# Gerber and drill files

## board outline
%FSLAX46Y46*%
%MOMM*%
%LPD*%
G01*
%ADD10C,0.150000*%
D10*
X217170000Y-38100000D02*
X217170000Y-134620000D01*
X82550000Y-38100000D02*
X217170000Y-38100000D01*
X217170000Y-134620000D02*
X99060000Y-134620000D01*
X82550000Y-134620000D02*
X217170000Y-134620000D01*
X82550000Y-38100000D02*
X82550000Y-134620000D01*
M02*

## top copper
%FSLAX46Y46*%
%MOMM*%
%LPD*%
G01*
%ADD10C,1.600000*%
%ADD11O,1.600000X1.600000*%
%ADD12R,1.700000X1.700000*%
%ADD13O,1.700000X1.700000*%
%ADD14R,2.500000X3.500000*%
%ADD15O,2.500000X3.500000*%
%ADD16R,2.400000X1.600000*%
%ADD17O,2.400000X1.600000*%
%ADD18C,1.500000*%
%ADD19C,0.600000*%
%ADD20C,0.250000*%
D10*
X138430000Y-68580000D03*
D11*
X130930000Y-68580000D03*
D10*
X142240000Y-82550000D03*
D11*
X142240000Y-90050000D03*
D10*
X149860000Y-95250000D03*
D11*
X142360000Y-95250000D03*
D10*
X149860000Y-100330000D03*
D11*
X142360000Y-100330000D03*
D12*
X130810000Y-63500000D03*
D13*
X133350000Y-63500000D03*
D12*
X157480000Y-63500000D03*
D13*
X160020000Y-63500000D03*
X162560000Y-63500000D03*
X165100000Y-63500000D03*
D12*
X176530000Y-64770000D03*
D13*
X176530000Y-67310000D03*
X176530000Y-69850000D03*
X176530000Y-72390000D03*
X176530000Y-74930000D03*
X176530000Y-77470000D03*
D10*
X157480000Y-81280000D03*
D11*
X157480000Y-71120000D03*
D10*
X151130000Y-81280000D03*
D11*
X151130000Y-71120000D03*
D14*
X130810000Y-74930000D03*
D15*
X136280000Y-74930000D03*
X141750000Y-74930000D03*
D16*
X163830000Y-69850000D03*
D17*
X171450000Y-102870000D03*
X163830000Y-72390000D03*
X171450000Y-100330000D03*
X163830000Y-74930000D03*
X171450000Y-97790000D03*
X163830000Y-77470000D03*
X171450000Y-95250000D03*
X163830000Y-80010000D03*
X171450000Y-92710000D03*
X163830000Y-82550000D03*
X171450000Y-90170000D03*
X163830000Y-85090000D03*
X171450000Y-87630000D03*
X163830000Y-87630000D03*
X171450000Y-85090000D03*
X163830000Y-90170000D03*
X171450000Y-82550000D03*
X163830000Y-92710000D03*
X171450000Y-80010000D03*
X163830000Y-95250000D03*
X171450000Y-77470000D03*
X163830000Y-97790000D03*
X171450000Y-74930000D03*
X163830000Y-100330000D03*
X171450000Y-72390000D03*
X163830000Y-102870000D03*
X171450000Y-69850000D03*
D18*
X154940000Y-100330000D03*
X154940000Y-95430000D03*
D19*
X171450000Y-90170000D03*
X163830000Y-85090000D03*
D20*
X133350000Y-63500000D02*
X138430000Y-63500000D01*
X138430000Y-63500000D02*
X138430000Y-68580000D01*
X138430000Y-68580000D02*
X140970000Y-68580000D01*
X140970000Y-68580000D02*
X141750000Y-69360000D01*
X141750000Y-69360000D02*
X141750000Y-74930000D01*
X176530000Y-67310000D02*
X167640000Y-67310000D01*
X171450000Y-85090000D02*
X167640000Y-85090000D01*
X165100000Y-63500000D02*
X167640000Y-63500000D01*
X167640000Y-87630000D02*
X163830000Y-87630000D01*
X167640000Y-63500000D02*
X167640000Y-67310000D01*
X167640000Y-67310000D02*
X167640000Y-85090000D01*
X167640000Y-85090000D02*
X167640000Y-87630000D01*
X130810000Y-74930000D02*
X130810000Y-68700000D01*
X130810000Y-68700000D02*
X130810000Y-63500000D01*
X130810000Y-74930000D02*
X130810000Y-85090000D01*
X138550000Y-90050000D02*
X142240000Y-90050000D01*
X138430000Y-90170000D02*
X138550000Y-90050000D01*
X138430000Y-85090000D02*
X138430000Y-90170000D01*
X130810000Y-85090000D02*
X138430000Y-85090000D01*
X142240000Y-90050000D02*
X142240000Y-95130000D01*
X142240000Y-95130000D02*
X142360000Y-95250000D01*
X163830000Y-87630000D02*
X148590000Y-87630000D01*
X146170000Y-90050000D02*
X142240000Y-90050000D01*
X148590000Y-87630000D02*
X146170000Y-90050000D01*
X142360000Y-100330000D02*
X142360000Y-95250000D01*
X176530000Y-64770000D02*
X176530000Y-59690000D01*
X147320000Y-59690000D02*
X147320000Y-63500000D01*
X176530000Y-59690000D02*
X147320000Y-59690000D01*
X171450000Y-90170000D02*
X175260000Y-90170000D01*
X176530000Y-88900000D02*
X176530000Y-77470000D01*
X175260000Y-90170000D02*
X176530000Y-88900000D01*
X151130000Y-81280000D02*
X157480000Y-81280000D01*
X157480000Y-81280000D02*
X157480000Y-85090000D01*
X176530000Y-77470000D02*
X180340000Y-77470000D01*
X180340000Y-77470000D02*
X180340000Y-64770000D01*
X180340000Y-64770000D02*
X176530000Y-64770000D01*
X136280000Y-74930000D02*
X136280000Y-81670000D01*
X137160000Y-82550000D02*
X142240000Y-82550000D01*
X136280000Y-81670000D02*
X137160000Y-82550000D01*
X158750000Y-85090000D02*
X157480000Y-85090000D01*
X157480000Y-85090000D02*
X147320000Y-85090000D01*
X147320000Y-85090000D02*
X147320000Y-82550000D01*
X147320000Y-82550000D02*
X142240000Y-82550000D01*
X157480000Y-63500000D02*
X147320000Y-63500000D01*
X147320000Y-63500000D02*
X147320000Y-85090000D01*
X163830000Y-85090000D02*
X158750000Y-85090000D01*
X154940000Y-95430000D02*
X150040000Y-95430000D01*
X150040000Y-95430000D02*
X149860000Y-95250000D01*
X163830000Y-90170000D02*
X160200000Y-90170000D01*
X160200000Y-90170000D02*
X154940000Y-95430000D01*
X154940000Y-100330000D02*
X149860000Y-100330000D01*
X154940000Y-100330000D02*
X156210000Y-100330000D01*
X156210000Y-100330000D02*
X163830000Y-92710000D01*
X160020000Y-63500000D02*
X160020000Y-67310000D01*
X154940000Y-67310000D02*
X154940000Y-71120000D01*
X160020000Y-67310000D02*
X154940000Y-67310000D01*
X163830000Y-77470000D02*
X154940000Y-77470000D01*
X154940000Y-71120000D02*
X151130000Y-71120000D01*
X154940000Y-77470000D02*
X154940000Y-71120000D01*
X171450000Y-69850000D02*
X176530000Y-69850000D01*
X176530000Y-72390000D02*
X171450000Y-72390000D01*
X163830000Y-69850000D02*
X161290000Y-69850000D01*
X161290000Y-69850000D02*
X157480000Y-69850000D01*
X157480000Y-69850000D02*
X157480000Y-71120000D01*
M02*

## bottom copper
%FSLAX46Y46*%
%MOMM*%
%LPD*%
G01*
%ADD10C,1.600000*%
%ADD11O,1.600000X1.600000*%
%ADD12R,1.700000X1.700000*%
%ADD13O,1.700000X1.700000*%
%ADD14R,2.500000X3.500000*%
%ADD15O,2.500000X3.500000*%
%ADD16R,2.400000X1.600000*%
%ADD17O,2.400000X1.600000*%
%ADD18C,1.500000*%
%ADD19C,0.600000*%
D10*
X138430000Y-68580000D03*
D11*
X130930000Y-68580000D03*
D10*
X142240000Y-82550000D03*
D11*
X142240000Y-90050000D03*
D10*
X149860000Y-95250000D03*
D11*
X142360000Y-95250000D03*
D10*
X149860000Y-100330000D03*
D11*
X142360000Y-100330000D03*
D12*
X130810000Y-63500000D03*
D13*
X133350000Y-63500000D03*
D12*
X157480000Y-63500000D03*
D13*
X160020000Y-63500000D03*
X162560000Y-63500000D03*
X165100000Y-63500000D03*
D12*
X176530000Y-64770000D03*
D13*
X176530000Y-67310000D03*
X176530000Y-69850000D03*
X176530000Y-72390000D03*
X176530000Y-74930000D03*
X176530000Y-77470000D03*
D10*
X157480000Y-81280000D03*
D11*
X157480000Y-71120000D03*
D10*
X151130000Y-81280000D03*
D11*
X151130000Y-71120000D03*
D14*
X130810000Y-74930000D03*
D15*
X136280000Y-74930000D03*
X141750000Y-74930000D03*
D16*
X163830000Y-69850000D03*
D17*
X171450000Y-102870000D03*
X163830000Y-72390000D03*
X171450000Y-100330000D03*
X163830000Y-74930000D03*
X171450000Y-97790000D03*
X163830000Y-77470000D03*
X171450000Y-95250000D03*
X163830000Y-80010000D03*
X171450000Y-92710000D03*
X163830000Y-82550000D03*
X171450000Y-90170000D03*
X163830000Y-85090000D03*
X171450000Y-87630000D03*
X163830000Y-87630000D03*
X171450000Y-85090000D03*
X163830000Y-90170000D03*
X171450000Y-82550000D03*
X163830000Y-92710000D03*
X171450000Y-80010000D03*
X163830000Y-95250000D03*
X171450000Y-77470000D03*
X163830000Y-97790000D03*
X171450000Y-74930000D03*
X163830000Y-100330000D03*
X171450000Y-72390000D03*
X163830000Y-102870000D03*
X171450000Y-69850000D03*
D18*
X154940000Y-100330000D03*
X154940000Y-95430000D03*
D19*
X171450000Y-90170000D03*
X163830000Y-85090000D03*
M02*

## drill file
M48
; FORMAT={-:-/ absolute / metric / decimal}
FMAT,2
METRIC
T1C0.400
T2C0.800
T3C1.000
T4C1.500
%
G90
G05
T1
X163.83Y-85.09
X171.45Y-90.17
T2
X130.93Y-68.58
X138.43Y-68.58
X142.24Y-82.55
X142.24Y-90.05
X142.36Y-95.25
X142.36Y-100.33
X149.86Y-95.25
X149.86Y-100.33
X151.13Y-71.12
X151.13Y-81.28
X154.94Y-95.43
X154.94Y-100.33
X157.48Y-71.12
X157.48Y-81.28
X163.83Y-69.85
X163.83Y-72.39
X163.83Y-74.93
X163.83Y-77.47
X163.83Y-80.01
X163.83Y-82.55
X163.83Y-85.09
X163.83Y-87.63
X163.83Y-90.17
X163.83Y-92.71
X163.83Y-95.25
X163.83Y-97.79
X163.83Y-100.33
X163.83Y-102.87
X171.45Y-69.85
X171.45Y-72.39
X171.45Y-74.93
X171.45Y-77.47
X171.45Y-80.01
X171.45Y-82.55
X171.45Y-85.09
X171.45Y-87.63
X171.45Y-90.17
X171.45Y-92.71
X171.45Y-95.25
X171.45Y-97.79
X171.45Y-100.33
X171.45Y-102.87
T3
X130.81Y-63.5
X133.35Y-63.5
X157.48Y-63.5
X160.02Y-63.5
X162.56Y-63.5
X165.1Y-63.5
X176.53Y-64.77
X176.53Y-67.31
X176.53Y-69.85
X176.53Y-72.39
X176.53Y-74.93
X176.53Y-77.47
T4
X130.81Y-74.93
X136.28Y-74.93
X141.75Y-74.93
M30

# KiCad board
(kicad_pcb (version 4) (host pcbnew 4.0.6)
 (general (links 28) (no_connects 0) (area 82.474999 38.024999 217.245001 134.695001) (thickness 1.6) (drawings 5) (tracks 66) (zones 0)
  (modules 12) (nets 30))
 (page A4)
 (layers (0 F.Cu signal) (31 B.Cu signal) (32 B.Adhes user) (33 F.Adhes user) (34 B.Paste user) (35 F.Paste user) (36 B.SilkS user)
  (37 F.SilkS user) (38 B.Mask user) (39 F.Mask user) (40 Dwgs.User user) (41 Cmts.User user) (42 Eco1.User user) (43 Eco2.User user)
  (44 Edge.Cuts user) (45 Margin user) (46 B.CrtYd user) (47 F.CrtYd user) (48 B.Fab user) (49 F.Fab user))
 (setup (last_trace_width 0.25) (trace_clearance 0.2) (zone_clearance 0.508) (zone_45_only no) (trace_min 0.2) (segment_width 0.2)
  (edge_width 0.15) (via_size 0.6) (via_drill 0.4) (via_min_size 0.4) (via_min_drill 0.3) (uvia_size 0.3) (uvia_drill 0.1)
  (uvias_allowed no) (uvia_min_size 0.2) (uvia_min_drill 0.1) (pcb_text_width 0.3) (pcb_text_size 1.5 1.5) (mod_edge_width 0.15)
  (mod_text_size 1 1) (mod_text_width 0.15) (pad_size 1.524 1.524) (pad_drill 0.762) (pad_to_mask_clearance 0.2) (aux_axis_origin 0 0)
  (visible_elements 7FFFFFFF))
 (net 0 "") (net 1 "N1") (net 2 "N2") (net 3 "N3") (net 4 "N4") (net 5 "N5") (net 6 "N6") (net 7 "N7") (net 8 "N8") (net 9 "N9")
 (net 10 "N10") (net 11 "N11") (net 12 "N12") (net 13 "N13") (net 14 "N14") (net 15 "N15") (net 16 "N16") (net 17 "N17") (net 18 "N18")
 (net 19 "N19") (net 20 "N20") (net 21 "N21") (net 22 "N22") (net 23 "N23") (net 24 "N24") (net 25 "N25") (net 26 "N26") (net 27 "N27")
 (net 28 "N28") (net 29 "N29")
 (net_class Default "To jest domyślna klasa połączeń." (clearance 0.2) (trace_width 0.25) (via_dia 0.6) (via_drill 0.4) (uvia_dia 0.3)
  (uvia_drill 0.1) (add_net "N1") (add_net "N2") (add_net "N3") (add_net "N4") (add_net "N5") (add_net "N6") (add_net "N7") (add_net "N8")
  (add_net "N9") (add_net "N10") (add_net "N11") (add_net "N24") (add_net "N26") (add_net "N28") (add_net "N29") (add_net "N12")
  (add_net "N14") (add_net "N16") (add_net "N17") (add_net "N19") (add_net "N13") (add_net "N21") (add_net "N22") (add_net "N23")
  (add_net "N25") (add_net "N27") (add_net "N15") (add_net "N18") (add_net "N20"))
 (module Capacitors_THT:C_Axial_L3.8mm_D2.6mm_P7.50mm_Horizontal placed (layer F.Cu) (at 138.43 68.58 180)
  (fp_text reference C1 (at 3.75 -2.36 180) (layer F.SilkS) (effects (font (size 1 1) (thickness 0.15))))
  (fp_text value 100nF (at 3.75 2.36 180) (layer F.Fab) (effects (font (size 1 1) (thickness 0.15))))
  (pad 1 thru_hole circle (at 0 0 180) (size 1.6 1.6) (drill 0.8) (layers *.Cu *.Mask) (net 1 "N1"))
  (pad 2 thru_hole oval (at 7.5 0 180) (size 1.6 1.6) (drill 0.8) (layers *.Cu *.Mask) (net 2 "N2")))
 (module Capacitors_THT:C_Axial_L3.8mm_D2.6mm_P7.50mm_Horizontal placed (layer F.Cu) (at 142.24 82.55 270)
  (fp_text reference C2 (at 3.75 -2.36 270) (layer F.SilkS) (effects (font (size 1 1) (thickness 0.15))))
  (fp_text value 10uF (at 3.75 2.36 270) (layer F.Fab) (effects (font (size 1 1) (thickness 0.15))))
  (pad 1 thru_hole circle (at 0 0 270) (size 1.6 1.6) (drill 0.8) (layers *.Cu *.Mask) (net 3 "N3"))
  (pad 2 thru_hole oval (at 7.5 0 270) (size 1.6 1.6) (drill 0.8) (layers *.Cu *.Mask) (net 2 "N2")))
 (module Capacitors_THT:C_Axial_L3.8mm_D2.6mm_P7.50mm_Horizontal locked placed (layer F.Cu) (at 149.86 95.25 180)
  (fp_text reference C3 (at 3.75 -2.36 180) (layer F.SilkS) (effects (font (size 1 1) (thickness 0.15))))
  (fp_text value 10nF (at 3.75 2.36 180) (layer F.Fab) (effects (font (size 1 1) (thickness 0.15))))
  (pad 1 thru_hole circle (at 0 0 180) (size 1.6 1.6) (drill 0.8) (layers *.Cu *.Mask) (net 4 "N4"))
  (pad 2 thru_hole oval (at 7.5 0 180) (size 1.6 1.6) (drill 0.8) (layers *.Cu *.Mask) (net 2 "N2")))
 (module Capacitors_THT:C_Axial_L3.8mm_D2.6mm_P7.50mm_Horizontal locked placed (layer F.Cu) (at 149.86 100.33 180)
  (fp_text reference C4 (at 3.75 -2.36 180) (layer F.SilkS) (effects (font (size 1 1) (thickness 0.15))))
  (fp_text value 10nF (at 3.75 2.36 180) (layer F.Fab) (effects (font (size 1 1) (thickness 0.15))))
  (pad 1 thru_hole circle (at 0 0 180) (size 1.6 1.6) (drill 0.8) (layers *.Cu *.Mask) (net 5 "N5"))
  (pad 2 thru_hole oval (at 7.5 0 180) (size 1.6 1.6) (drill 0.8) (layers *.Cu *.Mask) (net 2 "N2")))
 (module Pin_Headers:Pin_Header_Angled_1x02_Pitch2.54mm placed (layer F.Cu) (at 130.81 63.5 90)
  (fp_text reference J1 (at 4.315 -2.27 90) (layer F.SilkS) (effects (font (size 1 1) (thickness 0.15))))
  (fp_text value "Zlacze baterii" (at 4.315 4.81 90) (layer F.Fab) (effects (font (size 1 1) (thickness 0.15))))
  (pad 1 thru_hole rect (at 0 0 90) (size 1.7 1.7) (drill 1) (layers *.Cu *.Mask) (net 2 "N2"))
  (pad 2 thru_hole oval (at 0 2.54 90) (size 1.7 1.7) (drill 1) (layers *.Cu *.Mask) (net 1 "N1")))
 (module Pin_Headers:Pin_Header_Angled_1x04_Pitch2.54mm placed (layer F.Cu) (at 157.48 63.5 90)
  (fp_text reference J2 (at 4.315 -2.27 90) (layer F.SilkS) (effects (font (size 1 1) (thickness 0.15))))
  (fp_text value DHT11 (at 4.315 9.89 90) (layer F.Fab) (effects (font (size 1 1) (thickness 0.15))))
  (pad 1 thru_hole rect (at 0 0 90) (size 1.7 1.7) (drill 1) (layers *.Cu *.Mask) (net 3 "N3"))
  (pad 2 thru_hole oval (at 0 2.54 90) (size 1.7 1.7) (drill 1) (layers *.Cu *.Mask) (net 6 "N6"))
  (pad 3 thru_hole oval (at 0 5.08 90) (size 1.7 1.7) (drill 1) (layers *.Cu *.Mask) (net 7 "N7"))
  (pad 4 thru_hole oval (at 0 7.62 90) (size 1.7 1.7) (drill 1) (layers *.Cu *.Mask) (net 2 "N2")))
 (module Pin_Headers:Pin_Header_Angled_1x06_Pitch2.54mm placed (layer F.Cu) (at 176.53 64.77)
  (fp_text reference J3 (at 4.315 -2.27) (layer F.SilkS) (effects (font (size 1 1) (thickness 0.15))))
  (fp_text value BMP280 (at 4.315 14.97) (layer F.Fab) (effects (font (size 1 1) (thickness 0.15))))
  (pad 1 thru_hole rect (at 0 0) (size 1.7 1.7) (drill 1) (layers *.Cu *.Mask) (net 3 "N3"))
  (pad 2 thru_hole oval (at 0 2.54) (size 1.7 1.7) (drill 1) (layers *.Cu *.Mask) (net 2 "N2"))
  (pad 3 thru_hole oval (at 0 5.08) (size 1.7 1.7) (drill 1) (layers *.Cu *.Mask) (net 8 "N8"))
  (pad 4 thru_hole oval (at 0 7.62) (size 1.7 1.7) (drill 1) (layers *.Cu *.Mask) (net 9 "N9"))
  (pad 5 thru_hole oval (at 0 10.16) (size 1.7 1.7) (drill 1) (layers *.Cu *.Mask) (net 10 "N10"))
  (pad 6 thru_hole oval (at 0 12.7) (size 1.7 1.7) (drill 1) (layers *.Cu *.Mask) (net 3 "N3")))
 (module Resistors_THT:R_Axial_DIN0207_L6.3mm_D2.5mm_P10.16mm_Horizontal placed (layer F.Cu) (at 157.48 81.28 90)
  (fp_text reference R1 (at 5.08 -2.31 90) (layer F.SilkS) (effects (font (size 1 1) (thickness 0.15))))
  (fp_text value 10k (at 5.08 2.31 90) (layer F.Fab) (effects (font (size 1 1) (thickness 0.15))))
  (pad 1 thru_hole circle (at 0 0 90) (size 1.6 1.6) (drill 0.8) (layers *.Cu *.Mask) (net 3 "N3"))
  (pad 2 thru_hole oval (at 10.16 0 90) (size 1.6 1.6) (drill 0.8) (layers *.Cu *.Mask) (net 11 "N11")))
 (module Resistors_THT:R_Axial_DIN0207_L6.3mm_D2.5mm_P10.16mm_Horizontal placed (layer F.Cu) (at 151.13 81.28 90)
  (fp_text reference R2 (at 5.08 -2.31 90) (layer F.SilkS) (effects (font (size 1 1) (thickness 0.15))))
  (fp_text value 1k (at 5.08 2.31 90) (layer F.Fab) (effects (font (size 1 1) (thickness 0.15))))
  (pad 1 thru_hole circle (at 0 0 90) (size 1.6 1.6) (drill 0.8) (layers *.Cu *.Mask) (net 3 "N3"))
  (pad 2 thru_hole oval (at 10.16 0 90) (size 1.6 1.6) (drill 0.8) (layers *.Cu *.Mask) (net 6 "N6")))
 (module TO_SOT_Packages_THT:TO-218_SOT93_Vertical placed (layer F.Cu) (at 130.81 74.93)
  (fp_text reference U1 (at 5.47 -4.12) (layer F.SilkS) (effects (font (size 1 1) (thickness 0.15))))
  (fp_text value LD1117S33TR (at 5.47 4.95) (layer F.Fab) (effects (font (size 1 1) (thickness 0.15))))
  (pad 1 thru_hole rect (at 0 0) (size 2.5 3.5) (drill 1.5) (layers *.Cu *.Mask) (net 2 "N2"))
  (pad 2 thru_hole oval (at 5.47 0) (size 2.5 3.5) (drill 1.5) (layers *.Cu *.Mask) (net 3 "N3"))
  (pad 3 thru_hole oval (at 10.94 0) (size 2.5 3.5) (drill 1.5) (layers *.Cu *.Mask) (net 1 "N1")))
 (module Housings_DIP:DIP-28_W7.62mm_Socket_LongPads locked (layer F.Cu) (at 163.83 69.85)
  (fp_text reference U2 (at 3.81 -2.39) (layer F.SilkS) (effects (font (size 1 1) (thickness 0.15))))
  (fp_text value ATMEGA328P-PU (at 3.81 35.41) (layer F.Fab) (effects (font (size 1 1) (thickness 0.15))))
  (pad 1 thru_hole rect (at 0 0) (size 2.4 1.6) (drill 0.8) (layers *.Cu *.Mask) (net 11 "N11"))
  (pad 15 thru_hole oval (at 7.62 33.02) (size 2.4 1.6) (drill 0.8) (layers *.Cu *.Mask) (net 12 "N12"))
  (pad 2 thru_hole oval (at 0 2.54) (size 2.4 1.6) (drill 0.8) (layers *.Cu *.Mask) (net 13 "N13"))
  (pad 16 thru_hole oval (at 7.62 30.48) (size 2.4 1.6) (drill 0.8) (layers *.Cu *.Mask) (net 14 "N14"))
  (pad 3 thru_hole oval (at 0 5.08) (size 2.4 1.6) (drill 0.8) (layers *.Cu *.Mask) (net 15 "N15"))
  (pad 17 thru_hole oval (at 7.62 27.94) (size 2.4 1.6) (drill 0.8) (layers *.Cu *.Mask) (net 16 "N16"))
  (pad 4 thru_hole oval (at 0 7.62) (size 2.4 1.6) (drill 0.8) (layers *.Cu *.Mask) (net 6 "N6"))
  (pad 18 thru_hole oval (at 7.62 25.4) (size 2.4 1.6) (drill 0.8) (layers *.Cu *.Mask) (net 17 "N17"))
  (pad 5 thru_hole oval (at 0 10.16) (size 2.4 1.6) (drill 0.8) (layers *.Cu *.Mask) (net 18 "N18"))
  (pad 19 thru_hole oval (at 7.62 22.86) (size 2.4 1.6) (drill 0.8) (layers *.Cu *.Mask) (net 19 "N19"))
  (pad 6 thru_hole oval (at 0 12.7) (size 2.4 1.6) (drill 0.8) (layers *.Cu *.Mask) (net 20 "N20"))
  (pad 20 thru_hole oval (at 7.62 20.32) (size 2.4 1.6) (drill 0.8) (layers *.Cu *.Mask) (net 3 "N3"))
  (pad 7 thru_hole oval (at 0 15.24) (size 2.4 1.6) (drill 0.8) (layers *.Cu *.Mask) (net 3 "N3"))
  (pad 21 thru_hole oval (at 7.62 17.78) (size 2.4 1.6) (drill 0.8) (layers *.Cu *.Mask) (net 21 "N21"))
  (pad 8 thru_hole oval (at 0 17.78) (size 2.4 1.6) (drill 0.8) (layers *.Cu *.Mask) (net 2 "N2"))
  (pad 22 thru_hole oval (at 7.62 15.24) (size 2.4 1.6) (drill 0.8) (layers *.Cu *.Mask) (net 2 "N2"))
  (pad 9 thru_hole oval (at 0 20.32) (size 2.4 1.6) (drill 0.8) (layers *.Cu *.Mask) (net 4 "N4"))
  (pad 23 thru_hole oval (at 7.62 12.7) (size 2.4 1.6) (drill 0.8) (layers *.Cu *.Mask) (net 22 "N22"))
  (pad 10 thru_hole oval (at 0 22.86) (size 2.4 1.6) (drill 0.8) (layers *.Cu *.Mask) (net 5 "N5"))
  (pad 24 thru_hole oval (at 7.62 10.16) (size 2.4 1.6) (drill 0.8) (layers *.Cu *.Mask) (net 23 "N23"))
  (pad 11 thru_hole oval (at 0 25.4) (size 2.4 1.6) (drill 0.8) (layers *.Cu *.Mask) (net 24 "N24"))
  (pad 25 thru_hole oval (at 7.62 7.62) (size 2.4 1.6) (drill 0.8) (layers *.Cu *.Mask) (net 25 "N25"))
  (pad 12 thru_hole oval (at 0 27.94) (size 2.4 1.6) (drill 0.8) (layers *.Cu *.Mask) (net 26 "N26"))
  (pad 26 thru_hole oval (at 7.62 5.08) (size 2.4 1.6) (drill 0.8) (layers *.Cu *.Mask) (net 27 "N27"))
  (pad 13 thru_hole oval (at 0 30.48) (size 2.4 1.6) (drill 0.8) (layers *.Cu *.Mask) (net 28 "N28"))
  (pad 27 thru_hole oval (at 7.62 2.54) (size 2.4 1.6) (drill 0.8) (layers *.Cu *.Mask) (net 9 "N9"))
  (pad 14 thru_hole oval (at 0 33.02) (size 2.4 1.6) (drill 0.8) (layers *.Cu *.Mask) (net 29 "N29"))
  (pad 28 thru_hole oval (at 7.62 0) (size 2.4 1.6) (drill 0.8) (layers *.Cu *.Mask) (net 8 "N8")))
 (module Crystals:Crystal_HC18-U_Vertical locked (layer F.Cu) (at 154.94 100.33 90)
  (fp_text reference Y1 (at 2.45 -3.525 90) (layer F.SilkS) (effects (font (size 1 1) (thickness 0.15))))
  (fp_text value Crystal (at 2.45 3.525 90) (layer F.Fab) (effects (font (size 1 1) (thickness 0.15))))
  (pad 1 thru_hole circle (at 0 0 90) (size 1.5 1.5) (drill 0.8) (layers *.Cu *.Mask) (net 5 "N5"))
  (pad 2 thru_hole circle (at 4.9 0 90) (size 1.5 1.5) (drill 0.8) (layers *.Cu *.Mask) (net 4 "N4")))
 (gr_line (start 217.17 38.1) (end 217.17 134.62) (angle 90) (layer Edge.Cuts) (width 0.15))
 (gr_line (start 82.55 38.1) (end 217.17 38.1) (angle 90) (layer Edge.Cuts) (width 0.15))
 (gr_line (start 217.17 134.62) (end 99.06 134.62) (angle 90) (layer Edge.Cuts) (width 0.15))
 (gr_line (start 82.55 134.62) (end 217.17 134.62) (angle 90) (layer Edge.Cuts) (width 0.15))
 (gr_line (start 82.55 38.1) (end 82.55 134.62) (angle 90) (layer Edge.Cuts) (width 0.15))
 (segment (start 133.35 63.5) (end 138.43 63.5) (width 0.25) (layer F.Cu) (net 1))
 (segment (start 138.43 63.5) (end 138.43 68.58) (width 0.25) (layer F.Cu) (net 1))
 (segment (start 138.43 68.58) (end 140.97 68.58) (width 0.25) (layer F.Cu) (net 1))
 (segment (start 140.97 68.58) (end 141.75 69.36) (width 0.25) (layer F.Cu) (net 1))
 (segment (start 141.75 69.36) (end 141.75 74.93) (width 0.25) (layer F.Cu) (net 1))
 (segment (start 176.53 67.31) (end 167.64 67.31) (width 0.25) (layer F.Cu) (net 2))
 (segment (start 171.45 85.09) (end 167.64 85.09) (width 0.25) (layer F.Cu) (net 2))
 (segment (start 165.1 63.5) (end 167.64 63.5) (width 0.25) (layer F.Cu) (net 2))
 (segment (start 167.64 87.63) (end 163.83 87.63) (width 0.25) (layer F.Cu) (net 2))
 (segment (start 167.64 63.5) (end 167.64 67.31) (width 0.25) (layer F.Cu) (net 2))
 (segment (start 167.64 67.31) (end 167.64 85.09) (width 0.25) (layer F.Cu) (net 2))
 (segment (start 167.64 85.09) (end 167.64 87.63) (width 0.25) (layer F.Cu) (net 2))
 (segment (start 130.81 74.93) (end 130.81 68.7) (width 0.25) (layer F.Cu) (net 2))
 (segment (start 130.81 68.7) (end 130.81 63.5) (width 0.25) (layer F.Cu) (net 2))
 (segment (start 130.81 74.93) (end 130.81 85.09) (width 0.25) (layer F.Cu) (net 2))
 (segment (start 138.55 90.05) (end 142.24 90.05) (width 0.25) (layer F.Cu) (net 2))
 (segment (start 138.43 90.17) (end 138.55 90.05) (width 0.25) (layer F.Cu) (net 2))
 (segment (start 138.43 85.09) (end 138.43 90.17) (width 0.25) (layer F.Cu) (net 2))
 (segment (start 130.81 85.09) (end 138.43 85.09) (width 0.25) (layer F.Cu) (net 2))
 (segment (start 142.24 90.05) (end 142.24 95.13) (width 0.25) (layer F.Cu) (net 2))
 (segment (start 142.24 95.13) (end 142.36 95.25) (width 0.25) (layer F.Cu) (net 2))
 (segment (start 163.83 87.63) (end 148.59 87.63) (width 0.25) (layer F.Cu) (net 2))
 (segment (start 146.17 90.05) (end 142.24 90.05) (width 0.25) (layer F.Cu) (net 2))
 (segment (start 148.59 87.63) (end 146.17 90.05) (width 0.25) (layer F.Cu) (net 2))
 (segment (start 142.36 100.33) (end 142.36 95.25) (width 0.25) (layer F.Cu) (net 2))
 (segment (start 176.53 64.77) (end 176.53 59.69) (width 0.25) (layer F.Cu) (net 3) (status 400000))
 (segment (start 147.32 59.69) (end 147.32 63.5) (width 0.25) (layer F.Cu) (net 3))
 (segment (start 176.53 59.69) (end 147.32 59.69) (width 0.25) (layer F.Cu) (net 3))
 (segment (start 171.45 90.17) (end 175.26 90.17) (width 0.25) (layer F.Cu) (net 3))
 (segment (start 176.53 88.9) (end 176.53 77.47) (width 0.25) (layer F.Cu) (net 3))
 (segment (start 175.26 90.17) (end 176.53 88.9) (width 0.25) (layer F.Cu) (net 3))
 (segment (start 151.13 81.28) (end 157.48 81.28) (width 0.25) (layer F.Cu) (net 3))
 (segment (start 157.48 81.28) (end 157.48 85.09) (width 0.25) (layer F.Cu) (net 3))
 (via (at 171.45 90.17) (size 0.6) (drill 0.4) (layers F.Cu B.Cu) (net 3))
 (via (at 163.83 85.09) (size 0.6) (drill 0.4) (layers F.Cu B.Cu) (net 3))
 (segment (start 176.53 77.47) (end 180.34 77.47) (width 0.25) (layer F.Cu) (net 3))
 (segment (start 180.34 77.47) (end 180.34 64.77) (width 0.25) (layer F.Cu) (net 3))
 (segment (start 180.34 64.77) (end 176.53 64.77) (width 0.25) (layer F.Cu) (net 3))
 (segment (start 136.28 74.93) (end 136.28 81.67) (width 0.25) (layer F.Cu) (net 3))
 (segment (start 137.16 82.55) (end 142.24 82.55) (width 0.25) (layer F.Cu) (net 3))
 (segment (start 136.28 81.67) (end 137.16 82.55) (width 0.25) (layer F.Cu) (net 3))
 (segment (start 158.75 85.09) (end 157.48 85.09) (width 0.25) (layer F.Cu) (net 3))
 (segment (start 157.48 85.09) (end 147.32 85.09) (width 0.25) (layer F.Cu) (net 3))
 (segment (start 147.32 85.09) (end 147.32 82.55) (width 0.25) (layer F.Cu) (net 3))
 (segment (start 147.32 82.55) (end 142.24 82.55) (width 0.25) (layer F.Cu) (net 3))
 (segment (start 157.48 63.5) (end 147.32 63.5) (width 0.25) (layer F.Cu) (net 3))
 (segment (start 147.32 63.5) (end 147.32 85.09) (width 0.25) (layer F.Cu) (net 3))
 (segment (start 163.83 85.09) (end 158.75 85.09) (width 0.25) (layer F.Cu) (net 3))
 (segment (start 154.94 95.43) (end 150.04 95.43) (width 0.25) (layer F.Cu) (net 4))
 (segment (start 150.04 95.43) (end 149.86 95.25) (width 0.25) (layer F.Cu) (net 4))
 (segment (start 163.83 90.17) (end 160.2 90.17) (width 0.25) (layer F.Cu) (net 4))
 (segment (start 160.2 90.17) (end 154.94 95.43) (width 0.25) (layer F.Cu) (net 4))
 (segment (start 154.94 100.33) (end 149.86 100.33) (width 0.25) (layer F.Cu) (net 5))
 (segment (start 154.94 100.33) (end 156.21 100.33) (width 0.25) (layer F.Cu) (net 5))
 (segment (start 156.21 100.33) (end 163.83 92.71) (width 0.25) (layer F.Cu) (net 5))
 (segment (start 160.02 63.5) (end 160.02 67.31) (width 0.25) (layer F.Cu) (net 6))
 (segment (start 154.94 67.31) (end 154.94 71.12) (width 0.25) (layer F.Cu) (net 6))
 (segment (start 160.02 67.31) (end 154.94 67.31) (width 0.25) (layer F.Cu) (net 6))
 (segment (start 163.83 77.47) (end 154.94 77.47) (width 0.25) (layer F.Cu) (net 6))
 (segment (start 154.94 71.12) (end 151.13 71.12) (width 0.25) (layer F.Cu) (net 6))
 (segment (start 154.94 77.47) (end 154.94 71.12) (width 0.25) (layer F.Cu) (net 6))
 (segment (start 171.45 69.85) (end 176.53 69.85) (width 0.25) (layer F.Cu) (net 8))
 (segment (start 176.53 72.39) (end 171.45 72.39) (width 0.25) (layer F.Cu) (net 9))
 (segment (start 163.83 69.85) (end 161.29 69.85) (width 0.25) (layer F.Cu) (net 11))
 (segment (start 161.29 69.85) (end 157.48 69.85) (width 0.25) (layer F.Cu) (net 11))
 (segment (start 157.48 69.85) (end 157.48 71.12) (width 0.25) (layer F.Cu) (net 11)))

